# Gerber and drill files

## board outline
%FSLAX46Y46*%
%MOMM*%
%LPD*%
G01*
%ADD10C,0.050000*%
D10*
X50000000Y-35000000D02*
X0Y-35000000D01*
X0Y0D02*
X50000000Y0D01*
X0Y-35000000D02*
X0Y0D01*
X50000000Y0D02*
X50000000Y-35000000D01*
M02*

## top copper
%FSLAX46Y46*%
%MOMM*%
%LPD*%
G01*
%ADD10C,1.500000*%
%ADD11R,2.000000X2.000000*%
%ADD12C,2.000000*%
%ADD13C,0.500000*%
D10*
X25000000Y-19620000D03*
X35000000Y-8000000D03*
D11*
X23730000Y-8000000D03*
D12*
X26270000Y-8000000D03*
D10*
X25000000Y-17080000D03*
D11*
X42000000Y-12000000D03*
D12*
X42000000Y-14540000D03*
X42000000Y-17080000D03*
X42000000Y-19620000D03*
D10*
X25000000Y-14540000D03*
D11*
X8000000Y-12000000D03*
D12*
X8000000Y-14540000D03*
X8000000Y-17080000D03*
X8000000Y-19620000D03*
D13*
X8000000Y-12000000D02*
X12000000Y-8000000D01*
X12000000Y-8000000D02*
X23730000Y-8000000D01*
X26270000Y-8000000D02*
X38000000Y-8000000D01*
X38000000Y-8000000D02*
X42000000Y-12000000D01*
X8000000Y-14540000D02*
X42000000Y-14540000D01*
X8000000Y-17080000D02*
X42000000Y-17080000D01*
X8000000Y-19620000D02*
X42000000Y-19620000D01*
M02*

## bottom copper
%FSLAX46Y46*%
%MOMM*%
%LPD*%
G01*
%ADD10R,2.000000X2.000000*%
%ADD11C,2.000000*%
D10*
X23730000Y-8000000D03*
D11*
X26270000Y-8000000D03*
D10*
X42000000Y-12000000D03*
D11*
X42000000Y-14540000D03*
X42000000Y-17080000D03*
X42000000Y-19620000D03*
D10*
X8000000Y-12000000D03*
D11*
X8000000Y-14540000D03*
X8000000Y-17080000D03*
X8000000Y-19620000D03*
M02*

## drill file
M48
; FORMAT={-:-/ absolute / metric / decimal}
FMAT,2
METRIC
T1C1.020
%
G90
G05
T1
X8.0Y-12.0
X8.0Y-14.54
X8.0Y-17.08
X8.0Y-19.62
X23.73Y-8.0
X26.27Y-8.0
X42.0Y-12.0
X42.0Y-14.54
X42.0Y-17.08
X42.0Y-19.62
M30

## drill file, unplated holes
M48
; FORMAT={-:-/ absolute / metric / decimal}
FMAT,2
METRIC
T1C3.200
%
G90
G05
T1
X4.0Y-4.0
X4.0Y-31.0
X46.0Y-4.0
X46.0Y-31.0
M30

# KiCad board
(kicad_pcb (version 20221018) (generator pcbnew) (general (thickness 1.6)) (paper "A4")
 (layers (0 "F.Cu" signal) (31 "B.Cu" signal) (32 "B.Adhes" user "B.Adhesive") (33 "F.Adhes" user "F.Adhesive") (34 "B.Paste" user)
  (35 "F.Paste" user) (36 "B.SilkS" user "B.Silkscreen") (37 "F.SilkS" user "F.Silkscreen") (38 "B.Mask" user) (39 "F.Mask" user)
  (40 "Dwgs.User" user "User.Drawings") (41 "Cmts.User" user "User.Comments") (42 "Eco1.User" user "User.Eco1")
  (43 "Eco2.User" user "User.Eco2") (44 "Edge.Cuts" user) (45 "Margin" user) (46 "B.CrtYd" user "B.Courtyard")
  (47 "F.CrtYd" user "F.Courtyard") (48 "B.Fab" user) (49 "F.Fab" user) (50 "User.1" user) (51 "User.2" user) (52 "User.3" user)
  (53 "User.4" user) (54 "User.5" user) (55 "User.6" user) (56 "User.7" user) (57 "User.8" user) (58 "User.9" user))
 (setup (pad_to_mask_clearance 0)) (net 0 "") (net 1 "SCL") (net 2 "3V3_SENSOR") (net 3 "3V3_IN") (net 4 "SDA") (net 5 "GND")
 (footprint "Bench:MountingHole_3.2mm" (layer "F.Cu") (at 4 31)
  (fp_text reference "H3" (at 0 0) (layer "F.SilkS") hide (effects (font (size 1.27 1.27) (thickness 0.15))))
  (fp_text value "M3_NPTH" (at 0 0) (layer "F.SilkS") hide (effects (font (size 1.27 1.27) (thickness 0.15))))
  (pad "" np_thru_hole circle (at 0 0) (size 3.2 3.2) (drill 3.2) (layers "F&B.Cu" "*.Mask")))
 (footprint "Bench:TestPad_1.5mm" (layer "F.Cu") (at 25 19.62)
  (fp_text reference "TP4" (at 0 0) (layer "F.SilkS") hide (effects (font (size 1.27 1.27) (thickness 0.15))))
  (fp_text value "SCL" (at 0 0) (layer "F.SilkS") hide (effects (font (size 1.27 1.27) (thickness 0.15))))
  (pad "1" smd circle (at 0 0) (size 1.5 1.5) (layers "F.Cu" "F.Mask") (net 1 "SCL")))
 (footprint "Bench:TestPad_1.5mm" (layer "F.Cu") (at 35 8)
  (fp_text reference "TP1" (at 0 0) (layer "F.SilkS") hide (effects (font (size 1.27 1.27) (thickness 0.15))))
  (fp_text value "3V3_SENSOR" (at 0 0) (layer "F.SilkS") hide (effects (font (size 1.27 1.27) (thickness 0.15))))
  (pad "1" smd circle (at 0 0) (size 1.5 1.5) (layers "F.Cu" "F.Mask") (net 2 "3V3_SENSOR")))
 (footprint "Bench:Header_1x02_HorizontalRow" (layer "F.Cu") (at 23.73 8)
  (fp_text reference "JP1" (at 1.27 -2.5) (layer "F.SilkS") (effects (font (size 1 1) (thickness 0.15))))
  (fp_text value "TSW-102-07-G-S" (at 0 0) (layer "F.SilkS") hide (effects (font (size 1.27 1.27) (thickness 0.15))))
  (pad "1" thru_hole rect (at 0 0) (size 2 2) (drill 1.02) (layers "F&B.Cu" "*.Mask") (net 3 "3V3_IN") (thermal_bridge_angle 45))
  (pad "2" thru_hole circle (at 2.54 0) (size 2 2) (drill 1.02) (layers "F&B.Cu" "*.Mask") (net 2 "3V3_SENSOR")))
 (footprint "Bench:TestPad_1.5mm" (layer "F.Cu") (at 25 17.08)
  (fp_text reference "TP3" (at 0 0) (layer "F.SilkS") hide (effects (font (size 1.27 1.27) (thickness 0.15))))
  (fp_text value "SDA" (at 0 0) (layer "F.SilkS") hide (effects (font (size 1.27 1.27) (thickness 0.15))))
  (pad "1" smd circle (at 0 0) (size 1.5 1.5) (layers "F.Cu" "F.Mask") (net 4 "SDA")))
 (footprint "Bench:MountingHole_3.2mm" (layer "F.Cu") (at 46 4)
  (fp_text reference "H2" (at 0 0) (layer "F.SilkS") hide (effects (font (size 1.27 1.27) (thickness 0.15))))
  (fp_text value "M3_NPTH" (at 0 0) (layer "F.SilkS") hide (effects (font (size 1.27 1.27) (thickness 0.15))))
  (pad "" np_thru_hole circle (at 0 0) (size 3.2 3.2) (drill 3.2) (layers "F&B.Cu" "*.Mask")))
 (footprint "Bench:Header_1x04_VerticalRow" (layer "F.Cu") (at 42 12)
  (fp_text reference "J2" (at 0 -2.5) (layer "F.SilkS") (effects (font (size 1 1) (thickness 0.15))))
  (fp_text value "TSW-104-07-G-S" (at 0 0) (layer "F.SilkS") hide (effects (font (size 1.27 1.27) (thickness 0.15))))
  (pad "1" thru_hole rect (at 0 0) (size 2 2) (drill 1.02) (layers "F&B.Cu" "*.Mask") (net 2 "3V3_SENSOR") (thermal_bridge_angle 45))
  (pad "2" thru_hole circle (at 0 2.54) (size 2 2) (drill 1.02) (layers "F&B.Cu" "*.Mask") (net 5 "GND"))
  (pad "3" thru_hole circle (at 0 5.08) (size 2 2) (drill 1.02) (layers "F&B.Cu" "*.Mask") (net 4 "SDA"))
  (pad "4" thru_hole circle (at 0 7.62) (size 2 2) (drill 1.02) (layers "F&B.Cu" "*.Mask") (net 1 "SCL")))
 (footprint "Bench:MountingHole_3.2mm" (layer "F.Cu") (at 4 4)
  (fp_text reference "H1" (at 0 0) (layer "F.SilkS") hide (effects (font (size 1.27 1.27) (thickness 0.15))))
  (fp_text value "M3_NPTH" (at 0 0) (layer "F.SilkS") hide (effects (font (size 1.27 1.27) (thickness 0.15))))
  (pad "" np_thru_hole circle (at 0 0) (size 3.2 3.2) (drill 3.2) (layers "F&B.Cu" "*.Mask")))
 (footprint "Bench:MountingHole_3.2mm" (layer "F.Cu") (at 46 31)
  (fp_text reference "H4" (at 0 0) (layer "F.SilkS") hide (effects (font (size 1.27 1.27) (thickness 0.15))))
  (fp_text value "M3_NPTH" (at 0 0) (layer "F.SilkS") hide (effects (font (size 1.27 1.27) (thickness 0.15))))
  (pad "" np_thru_hole circle (at 0 0) (size 3.2 3.2) (drill 3.2) (layers "F&B.Cu" "*.Mask")))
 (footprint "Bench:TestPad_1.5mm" (layer "F.Cu") (at 25 14.54)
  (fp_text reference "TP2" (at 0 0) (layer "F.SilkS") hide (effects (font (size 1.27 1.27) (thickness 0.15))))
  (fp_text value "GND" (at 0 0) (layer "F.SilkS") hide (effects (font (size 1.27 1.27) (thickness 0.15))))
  (pad "1" smd circle (at 0 0) (size 1.5 1.5) (layers "F.Cu" "F.Mask") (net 5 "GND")))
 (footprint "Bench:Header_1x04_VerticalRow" (layer "F.Cu") (at 8 12)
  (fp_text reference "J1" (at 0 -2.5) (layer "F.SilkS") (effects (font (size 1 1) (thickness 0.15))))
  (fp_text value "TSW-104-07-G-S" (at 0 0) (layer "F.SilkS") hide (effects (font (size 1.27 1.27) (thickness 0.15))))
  (pad "1" thru_hole rect (at 0 0) (size 2 2) (drill 1.02) (layers "F&B.Cu" "*.Mask") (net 3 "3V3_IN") (thermal_bridge_angle 45))
  (pad "2" thru_hole circle (at 0 2.54) (size 2 2) (drill 1.02) (layers "F&B.Cu" "*.Mask") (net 5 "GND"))
  (pad "3" thru_hole circle (at 0 5.08) (size 2 2) (drill 1.02) (layers "F&B.Cu" "*.Mask") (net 4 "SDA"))
  (pad "4" thru_hole circle (at 0 7.62) (size 2 2) (drill 1.02) (layers "F&B.Cu" "*.Mask") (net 1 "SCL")))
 (gr_line (start 50 35) (end 0 35) (stroke (width 0.05) (type default)) (layer "Edge.Cuts"))
 (gr_line (start 0 0) (end 50 0) (stroke (width 0.05) (type default)) (layer "Edge.Cuts"))
 (gr_line (start 0 35) (end 0 0) (stroke (width 0.05) (type default)) (layer "Edge.Cuts"))
 (gr_line (start 50 0) (end 50 35) (stroke (width 0.05) (type default)) (layer "Edge.Cuts"))
 (segment (start 8 12) (end 12 8) (width 0.5) (layer "F.Cu") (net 3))
 (segment (start 12 8) (end 23.73 8) (width 0.5) (layer "F.Cu") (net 3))
 (segment (start 26.27 8) (end 38 8) (width 0.5) (layer "F.Cu") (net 2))
 (segment (start 38 8) (end 42 12) (width 0.5) (layer "F.Cu") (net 2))
 (segment (start 8 14.54) (end 42 14.54) (width 0.5) (layer "F.Cu") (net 5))
 (segment (start 8 17.08) (end 42 17.08) (width 0.5) (layer "F.Cu") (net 4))
 (segment (start 8 19.62) (end 42 19.62) (width 0.5) (layer "F.Cu") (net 1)))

